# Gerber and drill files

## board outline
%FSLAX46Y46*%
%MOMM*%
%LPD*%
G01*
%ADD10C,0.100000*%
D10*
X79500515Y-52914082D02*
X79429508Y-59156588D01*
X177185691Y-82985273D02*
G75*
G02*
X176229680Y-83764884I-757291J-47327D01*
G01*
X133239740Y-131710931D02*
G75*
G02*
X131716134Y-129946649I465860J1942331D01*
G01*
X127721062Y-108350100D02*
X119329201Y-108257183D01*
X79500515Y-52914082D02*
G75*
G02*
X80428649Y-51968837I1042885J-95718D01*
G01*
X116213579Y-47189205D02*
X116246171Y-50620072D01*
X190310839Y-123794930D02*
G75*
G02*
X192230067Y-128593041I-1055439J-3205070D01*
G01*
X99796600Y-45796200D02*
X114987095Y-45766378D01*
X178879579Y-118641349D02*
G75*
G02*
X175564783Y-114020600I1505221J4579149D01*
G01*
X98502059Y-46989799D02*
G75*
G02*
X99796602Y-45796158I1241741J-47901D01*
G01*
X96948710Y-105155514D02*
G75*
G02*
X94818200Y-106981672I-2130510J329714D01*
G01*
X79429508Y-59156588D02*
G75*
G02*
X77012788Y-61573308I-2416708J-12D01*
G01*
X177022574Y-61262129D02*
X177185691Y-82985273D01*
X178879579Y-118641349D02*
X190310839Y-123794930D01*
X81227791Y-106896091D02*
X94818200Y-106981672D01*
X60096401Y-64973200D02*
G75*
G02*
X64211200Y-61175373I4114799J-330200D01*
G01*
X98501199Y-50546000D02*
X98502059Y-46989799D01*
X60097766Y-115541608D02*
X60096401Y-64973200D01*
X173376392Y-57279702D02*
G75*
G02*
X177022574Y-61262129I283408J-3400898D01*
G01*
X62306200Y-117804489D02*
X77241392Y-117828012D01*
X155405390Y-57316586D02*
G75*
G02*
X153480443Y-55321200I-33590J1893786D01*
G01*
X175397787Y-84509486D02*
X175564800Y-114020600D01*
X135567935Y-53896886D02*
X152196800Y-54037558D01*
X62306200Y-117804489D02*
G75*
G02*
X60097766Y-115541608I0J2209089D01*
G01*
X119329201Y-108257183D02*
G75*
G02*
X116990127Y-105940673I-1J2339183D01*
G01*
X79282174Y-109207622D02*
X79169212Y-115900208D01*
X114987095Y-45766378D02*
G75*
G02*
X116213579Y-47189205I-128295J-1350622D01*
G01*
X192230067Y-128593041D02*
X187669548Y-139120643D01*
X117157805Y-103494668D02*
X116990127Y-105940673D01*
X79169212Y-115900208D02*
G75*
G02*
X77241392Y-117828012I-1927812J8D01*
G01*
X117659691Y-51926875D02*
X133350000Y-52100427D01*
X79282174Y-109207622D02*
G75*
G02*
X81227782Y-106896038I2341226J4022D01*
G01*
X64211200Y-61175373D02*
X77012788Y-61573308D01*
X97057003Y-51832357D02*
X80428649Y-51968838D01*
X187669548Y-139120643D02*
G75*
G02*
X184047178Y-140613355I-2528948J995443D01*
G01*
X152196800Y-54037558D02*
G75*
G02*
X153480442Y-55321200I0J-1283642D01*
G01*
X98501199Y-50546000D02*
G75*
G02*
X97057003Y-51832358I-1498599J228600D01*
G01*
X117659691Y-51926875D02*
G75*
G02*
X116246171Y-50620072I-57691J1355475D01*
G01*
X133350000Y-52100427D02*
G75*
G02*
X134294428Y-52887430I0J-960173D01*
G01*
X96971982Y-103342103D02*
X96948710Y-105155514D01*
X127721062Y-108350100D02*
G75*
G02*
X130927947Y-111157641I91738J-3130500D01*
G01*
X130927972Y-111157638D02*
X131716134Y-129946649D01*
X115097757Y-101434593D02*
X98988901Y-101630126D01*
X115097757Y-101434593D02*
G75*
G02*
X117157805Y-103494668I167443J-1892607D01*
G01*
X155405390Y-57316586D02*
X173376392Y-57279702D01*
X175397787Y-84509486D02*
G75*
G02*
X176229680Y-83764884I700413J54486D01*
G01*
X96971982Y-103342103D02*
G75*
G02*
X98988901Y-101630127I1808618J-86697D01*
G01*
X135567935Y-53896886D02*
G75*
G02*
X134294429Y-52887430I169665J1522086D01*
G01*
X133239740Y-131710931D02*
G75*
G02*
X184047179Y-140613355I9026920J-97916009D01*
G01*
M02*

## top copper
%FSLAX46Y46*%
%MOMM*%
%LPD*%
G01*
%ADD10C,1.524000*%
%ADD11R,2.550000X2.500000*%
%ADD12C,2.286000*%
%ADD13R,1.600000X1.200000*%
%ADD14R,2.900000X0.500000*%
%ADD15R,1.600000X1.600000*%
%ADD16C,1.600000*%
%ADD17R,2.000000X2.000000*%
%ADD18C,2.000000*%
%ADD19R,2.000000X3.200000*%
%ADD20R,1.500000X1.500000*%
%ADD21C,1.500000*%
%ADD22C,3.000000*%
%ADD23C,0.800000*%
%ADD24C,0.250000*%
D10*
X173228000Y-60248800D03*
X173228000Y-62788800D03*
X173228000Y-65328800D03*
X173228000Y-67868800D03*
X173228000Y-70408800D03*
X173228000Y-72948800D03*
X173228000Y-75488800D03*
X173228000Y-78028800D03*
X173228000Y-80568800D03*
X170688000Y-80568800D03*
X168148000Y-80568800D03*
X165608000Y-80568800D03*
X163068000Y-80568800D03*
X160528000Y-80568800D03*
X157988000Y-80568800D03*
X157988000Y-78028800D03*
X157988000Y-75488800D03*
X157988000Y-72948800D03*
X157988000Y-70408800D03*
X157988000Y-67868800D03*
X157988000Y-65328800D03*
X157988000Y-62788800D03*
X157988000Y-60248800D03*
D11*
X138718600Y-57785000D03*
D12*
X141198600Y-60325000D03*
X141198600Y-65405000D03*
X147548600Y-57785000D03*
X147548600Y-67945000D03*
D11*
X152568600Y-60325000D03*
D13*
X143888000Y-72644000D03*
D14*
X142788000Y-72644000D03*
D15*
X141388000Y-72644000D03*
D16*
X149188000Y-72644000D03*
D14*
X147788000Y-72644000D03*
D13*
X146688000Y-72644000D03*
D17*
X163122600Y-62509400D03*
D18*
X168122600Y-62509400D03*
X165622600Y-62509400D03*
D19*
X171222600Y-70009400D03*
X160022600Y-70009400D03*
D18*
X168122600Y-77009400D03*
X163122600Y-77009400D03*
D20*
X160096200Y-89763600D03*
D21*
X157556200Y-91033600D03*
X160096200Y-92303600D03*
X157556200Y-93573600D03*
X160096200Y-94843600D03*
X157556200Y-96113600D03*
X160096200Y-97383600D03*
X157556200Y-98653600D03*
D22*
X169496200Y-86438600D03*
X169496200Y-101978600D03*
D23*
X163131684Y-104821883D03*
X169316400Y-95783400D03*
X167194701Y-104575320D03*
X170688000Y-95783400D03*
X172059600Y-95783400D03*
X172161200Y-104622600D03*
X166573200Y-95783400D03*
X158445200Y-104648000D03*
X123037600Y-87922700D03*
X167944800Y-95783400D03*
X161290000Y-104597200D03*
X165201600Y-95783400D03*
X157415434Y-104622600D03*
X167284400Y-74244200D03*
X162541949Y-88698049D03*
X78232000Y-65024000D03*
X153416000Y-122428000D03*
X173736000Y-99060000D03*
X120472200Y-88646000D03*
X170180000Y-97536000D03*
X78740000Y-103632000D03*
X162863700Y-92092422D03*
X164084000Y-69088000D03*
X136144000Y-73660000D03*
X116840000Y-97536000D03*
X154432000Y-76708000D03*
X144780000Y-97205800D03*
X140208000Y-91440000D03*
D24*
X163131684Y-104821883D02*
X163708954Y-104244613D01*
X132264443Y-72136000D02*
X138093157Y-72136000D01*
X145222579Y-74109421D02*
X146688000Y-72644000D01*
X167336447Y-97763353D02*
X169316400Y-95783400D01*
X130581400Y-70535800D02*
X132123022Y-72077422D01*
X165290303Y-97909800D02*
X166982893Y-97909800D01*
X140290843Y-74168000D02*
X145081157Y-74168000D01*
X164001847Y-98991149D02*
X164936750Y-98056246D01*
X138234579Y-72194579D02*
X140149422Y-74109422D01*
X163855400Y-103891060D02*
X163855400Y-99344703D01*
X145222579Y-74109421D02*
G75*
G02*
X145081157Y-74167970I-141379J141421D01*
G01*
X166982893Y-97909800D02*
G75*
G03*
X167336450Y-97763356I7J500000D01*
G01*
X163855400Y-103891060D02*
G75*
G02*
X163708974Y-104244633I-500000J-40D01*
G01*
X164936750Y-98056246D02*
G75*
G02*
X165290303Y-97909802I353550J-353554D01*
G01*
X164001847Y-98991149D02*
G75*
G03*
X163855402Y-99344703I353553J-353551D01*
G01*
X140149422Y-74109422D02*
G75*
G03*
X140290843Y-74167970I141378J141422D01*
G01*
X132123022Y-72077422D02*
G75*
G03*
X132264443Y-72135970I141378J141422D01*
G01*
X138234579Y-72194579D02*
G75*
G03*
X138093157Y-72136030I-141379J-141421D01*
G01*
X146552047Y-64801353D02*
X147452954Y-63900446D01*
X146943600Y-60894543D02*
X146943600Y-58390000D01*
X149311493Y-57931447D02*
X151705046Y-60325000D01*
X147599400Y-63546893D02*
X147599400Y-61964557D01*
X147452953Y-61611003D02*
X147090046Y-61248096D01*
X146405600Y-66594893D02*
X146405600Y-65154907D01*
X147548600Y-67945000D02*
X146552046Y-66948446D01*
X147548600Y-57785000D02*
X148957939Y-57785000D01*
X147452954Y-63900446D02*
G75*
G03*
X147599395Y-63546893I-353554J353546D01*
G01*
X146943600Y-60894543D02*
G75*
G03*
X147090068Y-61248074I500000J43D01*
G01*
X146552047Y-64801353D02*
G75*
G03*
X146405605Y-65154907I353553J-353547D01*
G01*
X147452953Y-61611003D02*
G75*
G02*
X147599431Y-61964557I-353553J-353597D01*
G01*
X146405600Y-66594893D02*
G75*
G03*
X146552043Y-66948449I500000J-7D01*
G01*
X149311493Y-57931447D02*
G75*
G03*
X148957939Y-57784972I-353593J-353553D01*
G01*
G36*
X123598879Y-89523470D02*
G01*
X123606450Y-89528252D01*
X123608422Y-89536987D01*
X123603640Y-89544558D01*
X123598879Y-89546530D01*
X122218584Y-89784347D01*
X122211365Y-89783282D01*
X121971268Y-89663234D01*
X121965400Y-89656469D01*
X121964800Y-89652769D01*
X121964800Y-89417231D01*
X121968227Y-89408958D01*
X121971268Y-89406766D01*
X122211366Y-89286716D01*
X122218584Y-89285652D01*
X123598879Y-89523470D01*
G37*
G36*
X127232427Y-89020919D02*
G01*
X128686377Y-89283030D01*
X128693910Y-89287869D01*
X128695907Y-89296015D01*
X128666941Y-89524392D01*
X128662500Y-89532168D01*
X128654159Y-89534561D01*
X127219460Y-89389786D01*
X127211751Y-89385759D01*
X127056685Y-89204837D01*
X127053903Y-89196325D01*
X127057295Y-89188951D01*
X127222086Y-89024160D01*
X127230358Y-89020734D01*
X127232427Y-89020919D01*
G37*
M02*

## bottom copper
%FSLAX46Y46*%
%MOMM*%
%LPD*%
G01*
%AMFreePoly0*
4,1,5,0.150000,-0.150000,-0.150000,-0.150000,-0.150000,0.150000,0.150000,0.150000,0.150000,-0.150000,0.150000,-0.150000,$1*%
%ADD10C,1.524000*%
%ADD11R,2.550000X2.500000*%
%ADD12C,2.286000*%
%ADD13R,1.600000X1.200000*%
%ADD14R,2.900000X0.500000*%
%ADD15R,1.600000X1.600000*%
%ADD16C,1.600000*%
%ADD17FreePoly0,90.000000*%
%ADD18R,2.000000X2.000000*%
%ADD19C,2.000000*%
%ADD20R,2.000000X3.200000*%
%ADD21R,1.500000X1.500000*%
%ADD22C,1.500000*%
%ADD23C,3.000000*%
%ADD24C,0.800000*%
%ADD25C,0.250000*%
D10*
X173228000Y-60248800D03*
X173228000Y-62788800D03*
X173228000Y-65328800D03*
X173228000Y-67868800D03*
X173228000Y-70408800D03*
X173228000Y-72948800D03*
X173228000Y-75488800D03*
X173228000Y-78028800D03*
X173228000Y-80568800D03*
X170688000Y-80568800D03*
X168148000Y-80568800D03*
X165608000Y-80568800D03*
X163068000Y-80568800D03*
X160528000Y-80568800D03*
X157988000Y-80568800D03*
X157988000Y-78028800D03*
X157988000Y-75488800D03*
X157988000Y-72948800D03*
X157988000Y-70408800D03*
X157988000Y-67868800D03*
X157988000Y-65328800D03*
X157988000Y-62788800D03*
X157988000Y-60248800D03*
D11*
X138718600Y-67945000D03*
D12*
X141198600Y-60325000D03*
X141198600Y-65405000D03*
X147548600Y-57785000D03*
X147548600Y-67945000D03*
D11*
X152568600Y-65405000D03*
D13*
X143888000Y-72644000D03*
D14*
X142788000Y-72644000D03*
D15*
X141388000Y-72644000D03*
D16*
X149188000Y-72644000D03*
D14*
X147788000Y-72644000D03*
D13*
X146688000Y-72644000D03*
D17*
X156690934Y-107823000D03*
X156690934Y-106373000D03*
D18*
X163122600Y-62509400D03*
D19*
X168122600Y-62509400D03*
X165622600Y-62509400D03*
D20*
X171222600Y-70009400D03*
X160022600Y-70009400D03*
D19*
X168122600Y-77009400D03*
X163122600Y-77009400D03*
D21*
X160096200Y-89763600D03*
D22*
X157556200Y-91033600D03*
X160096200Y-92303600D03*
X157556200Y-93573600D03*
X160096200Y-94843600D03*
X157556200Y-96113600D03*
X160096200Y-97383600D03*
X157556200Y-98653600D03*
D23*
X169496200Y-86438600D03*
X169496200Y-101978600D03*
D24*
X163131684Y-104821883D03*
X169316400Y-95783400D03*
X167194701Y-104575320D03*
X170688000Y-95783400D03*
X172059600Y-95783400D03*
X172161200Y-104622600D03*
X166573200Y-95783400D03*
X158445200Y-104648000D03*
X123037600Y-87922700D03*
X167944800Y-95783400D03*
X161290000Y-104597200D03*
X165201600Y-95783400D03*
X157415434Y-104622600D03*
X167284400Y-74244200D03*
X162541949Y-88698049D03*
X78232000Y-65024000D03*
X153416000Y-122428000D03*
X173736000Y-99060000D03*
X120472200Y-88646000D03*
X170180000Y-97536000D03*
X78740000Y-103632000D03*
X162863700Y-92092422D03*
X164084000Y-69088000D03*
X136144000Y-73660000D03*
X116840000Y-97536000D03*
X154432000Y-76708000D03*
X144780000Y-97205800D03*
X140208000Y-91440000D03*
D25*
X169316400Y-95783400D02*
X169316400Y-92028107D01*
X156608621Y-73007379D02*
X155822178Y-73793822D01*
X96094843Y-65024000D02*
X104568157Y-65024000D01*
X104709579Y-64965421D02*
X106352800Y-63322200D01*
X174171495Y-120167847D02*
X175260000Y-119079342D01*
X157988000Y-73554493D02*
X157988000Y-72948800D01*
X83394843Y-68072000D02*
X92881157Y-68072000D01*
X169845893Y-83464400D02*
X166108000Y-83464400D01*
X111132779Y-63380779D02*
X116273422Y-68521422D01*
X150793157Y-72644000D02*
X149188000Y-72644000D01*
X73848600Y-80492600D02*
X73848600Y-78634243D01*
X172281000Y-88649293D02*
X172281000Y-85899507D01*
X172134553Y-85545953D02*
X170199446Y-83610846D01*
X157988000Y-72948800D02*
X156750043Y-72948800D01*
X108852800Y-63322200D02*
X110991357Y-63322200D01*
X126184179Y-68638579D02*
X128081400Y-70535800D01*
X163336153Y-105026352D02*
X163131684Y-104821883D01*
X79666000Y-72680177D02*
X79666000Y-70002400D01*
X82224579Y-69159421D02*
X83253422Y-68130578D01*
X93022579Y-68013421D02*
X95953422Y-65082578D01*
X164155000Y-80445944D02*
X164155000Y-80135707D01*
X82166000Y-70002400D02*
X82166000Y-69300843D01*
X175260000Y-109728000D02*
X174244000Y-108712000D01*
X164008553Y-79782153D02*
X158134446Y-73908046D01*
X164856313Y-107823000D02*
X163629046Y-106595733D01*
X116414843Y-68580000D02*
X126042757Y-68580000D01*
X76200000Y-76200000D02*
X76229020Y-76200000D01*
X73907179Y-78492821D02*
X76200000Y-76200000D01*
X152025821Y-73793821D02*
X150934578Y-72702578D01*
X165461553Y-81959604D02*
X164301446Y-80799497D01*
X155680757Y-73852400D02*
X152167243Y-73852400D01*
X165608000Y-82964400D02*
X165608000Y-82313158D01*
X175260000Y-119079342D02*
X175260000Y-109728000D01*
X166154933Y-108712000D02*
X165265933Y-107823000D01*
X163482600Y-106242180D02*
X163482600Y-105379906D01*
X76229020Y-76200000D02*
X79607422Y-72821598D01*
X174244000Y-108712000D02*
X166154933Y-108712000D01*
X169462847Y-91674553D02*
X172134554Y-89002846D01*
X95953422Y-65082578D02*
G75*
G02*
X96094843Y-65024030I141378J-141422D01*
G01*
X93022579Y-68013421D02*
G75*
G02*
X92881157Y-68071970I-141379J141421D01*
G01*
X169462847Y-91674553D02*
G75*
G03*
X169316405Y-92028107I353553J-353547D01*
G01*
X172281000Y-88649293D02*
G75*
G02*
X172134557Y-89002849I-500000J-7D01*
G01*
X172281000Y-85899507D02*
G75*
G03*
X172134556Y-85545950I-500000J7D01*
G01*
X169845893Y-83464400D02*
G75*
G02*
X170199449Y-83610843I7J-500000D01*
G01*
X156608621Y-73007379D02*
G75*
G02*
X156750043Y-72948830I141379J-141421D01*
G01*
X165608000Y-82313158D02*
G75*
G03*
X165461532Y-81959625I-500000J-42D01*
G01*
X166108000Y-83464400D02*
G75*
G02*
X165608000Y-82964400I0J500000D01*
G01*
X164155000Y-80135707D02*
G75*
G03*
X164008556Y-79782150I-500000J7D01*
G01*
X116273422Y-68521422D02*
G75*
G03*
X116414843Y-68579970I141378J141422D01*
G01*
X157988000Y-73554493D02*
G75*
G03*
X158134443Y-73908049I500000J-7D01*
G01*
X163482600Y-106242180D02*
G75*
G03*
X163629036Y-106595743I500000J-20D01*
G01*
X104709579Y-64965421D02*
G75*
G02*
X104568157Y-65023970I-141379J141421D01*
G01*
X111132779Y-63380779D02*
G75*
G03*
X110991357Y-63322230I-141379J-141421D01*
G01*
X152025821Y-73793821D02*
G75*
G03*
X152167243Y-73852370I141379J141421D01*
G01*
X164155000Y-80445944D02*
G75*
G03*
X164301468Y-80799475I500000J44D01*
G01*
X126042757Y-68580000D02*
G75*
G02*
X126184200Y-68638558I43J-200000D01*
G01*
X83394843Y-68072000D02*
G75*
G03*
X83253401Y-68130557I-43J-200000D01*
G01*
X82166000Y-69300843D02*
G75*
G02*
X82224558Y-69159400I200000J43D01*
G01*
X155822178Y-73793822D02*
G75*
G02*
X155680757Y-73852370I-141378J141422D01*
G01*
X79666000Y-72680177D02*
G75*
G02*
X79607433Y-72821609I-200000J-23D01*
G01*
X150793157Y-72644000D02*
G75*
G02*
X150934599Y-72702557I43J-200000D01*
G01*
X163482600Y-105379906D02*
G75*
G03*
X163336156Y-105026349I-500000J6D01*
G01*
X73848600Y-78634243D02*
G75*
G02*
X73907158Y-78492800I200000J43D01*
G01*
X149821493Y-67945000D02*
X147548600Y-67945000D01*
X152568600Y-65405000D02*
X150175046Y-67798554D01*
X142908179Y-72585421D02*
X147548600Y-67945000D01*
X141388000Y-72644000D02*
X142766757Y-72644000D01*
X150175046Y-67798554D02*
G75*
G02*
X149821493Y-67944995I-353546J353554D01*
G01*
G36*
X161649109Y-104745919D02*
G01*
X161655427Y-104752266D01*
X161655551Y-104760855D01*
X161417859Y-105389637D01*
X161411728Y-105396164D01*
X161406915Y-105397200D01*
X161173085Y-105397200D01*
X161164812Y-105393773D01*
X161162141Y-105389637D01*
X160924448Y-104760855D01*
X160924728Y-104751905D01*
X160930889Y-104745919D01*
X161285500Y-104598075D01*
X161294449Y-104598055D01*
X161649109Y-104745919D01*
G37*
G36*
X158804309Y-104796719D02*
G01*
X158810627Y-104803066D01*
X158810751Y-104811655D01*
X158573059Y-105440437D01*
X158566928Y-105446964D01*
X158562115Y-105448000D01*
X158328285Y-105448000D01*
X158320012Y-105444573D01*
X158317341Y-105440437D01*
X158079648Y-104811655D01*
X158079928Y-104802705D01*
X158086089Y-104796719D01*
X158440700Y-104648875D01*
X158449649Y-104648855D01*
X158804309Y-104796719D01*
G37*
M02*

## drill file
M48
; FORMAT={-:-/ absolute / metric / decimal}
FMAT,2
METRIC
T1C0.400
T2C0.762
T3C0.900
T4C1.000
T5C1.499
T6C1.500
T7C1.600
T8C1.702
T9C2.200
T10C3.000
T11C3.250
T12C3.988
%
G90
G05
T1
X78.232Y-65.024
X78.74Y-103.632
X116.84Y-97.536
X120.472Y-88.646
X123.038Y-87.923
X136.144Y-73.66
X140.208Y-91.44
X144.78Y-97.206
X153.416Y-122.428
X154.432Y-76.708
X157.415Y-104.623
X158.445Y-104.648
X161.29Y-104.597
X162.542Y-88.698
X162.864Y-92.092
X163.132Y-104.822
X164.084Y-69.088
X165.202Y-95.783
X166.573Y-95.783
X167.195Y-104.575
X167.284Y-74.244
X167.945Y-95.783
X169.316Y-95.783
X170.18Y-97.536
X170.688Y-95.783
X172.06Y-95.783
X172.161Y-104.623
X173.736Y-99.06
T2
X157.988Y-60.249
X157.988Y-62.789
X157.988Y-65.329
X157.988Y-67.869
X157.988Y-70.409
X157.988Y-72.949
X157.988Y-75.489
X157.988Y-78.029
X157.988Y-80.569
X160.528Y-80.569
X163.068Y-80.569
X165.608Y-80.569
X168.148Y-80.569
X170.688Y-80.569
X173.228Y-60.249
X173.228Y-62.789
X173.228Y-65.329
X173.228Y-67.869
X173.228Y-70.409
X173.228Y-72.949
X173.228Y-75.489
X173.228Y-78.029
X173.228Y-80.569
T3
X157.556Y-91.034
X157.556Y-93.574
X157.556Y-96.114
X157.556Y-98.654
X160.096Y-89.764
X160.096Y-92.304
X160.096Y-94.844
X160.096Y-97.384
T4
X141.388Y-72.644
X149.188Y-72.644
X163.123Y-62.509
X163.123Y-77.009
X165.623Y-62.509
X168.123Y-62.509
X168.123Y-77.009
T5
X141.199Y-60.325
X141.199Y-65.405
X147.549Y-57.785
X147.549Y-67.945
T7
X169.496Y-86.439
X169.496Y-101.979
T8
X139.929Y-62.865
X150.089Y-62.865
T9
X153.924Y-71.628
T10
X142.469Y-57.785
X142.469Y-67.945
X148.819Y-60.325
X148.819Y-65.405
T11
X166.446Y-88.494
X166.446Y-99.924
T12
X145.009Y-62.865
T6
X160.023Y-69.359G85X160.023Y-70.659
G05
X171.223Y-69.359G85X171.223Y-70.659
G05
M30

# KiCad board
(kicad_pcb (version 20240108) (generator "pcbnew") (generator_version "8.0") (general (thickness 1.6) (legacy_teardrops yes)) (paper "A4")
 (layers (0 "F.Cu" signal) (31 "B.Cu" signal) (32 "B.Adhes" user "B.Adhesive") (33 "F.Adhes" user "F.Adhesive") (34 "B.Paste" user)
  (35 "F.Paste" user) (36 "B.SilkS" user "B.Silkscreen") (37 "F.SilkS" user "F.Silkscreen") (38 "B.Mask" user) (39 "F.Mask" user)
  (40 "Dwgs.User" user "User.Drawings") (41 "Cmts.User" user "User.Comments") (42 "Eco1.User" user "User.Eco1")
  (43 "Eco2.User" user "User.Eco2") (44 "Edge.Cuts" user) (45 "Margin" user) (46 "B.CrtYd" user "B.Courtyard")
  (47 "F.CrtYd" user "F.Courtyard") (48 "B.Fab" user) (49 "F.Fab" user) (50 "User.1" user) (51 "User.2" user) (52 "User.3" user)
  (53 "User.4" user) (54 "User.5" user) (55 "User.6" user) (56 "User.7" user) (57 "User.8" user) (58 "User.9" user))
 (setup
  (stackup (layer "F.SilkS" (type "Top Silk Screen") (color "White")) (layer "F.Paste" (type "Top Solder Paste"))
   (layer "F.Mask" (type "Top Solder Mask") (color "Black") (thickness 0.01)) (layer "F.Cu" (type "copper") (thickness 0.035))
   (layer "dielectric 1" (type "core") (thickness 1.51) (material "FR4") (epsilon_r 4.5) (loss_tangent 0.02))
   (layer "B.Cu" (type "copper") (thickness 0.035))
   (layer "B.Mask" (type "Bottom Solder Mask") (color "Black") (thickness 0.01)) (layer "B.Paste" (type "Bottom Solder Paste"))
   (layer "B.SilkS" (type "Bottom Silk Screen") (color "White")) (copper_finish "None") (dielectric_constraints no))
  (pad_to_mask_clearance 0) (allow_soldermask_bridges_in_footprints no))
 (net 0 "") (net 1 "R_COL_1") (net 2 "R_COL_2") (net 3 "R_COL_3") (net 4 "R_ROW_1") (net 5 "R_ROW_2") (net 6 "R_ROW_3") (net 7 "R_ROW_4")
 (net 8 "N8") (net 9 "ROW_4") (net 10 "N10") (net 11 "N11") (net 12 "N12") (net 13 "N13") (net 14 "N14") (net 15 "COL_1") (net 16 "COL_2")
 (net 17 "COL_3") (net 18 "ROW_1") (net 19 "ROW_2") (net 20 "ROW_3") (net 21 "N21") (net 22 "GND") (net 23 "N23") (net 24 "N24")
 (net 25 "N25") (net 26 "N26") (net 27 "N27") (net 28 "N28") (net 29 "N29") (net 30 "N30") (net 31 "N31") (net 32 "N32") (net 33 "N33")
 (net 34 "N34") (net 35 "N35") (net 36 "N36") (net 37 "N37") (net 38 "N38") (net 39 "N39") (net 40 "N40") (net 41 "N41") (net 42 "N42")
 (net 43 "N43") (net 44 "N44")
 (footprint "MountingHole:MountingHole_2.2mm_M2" (layer "F.Cu") (at 153.924 71.628)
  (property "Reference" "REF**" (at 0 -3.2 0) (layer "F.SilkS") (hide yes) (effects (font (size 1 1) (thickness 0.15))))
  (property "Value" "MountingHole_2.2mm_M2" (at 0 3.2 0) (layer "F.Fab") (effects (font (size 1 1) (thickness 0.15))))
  (pad "" np_thru_hole circle (at 0 0) (size 2.2 2.2) (drill 2.2) (layers "*.Cu" "*.Mask")))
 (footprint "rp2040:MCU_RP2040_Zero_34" (layer "F.Cu") (at 163.068 67.8688)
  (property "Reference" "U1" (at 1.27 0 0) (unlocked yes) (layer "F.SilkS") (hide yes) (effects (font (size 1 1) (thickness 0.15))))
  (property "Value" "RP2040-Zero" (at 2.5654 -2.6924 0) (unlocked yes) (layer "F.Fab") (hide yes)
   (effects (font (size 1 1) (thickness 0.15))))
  (pad "0" thru_hole circle (at 10.16 -7.62) (size 1.524 1.524) (drill 0.762) (layers "*.Cu" "*.Mask") (remove_unused_layers no)
   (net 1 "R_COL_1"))
  (pad "1" thru_hole circle (at 10.16 -5.08) (size 1.524 1.524) (drill 0.762) (layers "*.Cu" "*.Mask") (remove_unused_layers no)
   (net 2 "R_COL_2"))
  (pad "2" thru_hole circle (at 10.16 -2.54) (size 1.524 1.524) (drill 0.762) (layers "*.Cu" "*.Mask") (remove_unused_layers no)
   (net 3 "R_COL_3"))
  (pad "3" thru_hole circle (at 10.16 0) (size 1.524 1.524) (drill 0.762) (layers "*.Cu" "*.Mask") (remove_unused_layers no)
   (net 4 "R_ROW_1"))
  (pad "4" thru_hole circle (at 10.16 2.54) (size 1.524 1.524) (drill 0.762) (layers "*.Cu" "*.Mask") (remove_unused_layers no)
   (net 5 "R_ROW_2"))
  (pad "5" thru_hole circle (at 10.16 5.08) (size 1.524 1.524) (drill 0.762) (layers "*.Cu" "*.Mask") (remove_unused_layers no)
   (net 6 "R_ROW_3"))
  (pad "6" thru_hole circle (at 10.16 7.62) (size 1.524 1.524) (drill 0.762) (layers "*.Cu" "*.Mask") (remove_unused_layers no)
   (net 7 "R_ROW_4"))
  (pad "7" thru_hole circle (at 10.16 10.16) (size 1.524 1.524) (drill 0.762) (layers "*.Cu" "*.Mask") (remove_unused_layers no)
   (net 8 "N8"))
  (pad "8" thru_hole circle (at 10.16 12.7) (size 1.524 1.524) (drill 0.762) (layers "*.Cu" "*.Mask") (remove_unused_layers no)
   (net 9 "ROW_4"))
  (pad "9" thru_hole circle (at 7.62 12.7) (size 1.524 1.524) (drill 0.762) (layers "*.Cu" "*.Mask") (remove_unused_layers no)
   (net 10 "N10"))
  (pad "10" thru_hole circle (at 5.08 12.7) (size 1.524 1.524) (drill 0.762) (layers "*.Cu" "*.Mask") (remove_unused_layers no)
   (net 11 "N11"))
  (pad "11" thru_hole circle (at 2.54 12.7) (size 1.524 1.524) (drill 0.762) (layers "*.Cu" "*.Mask") (remove_unused_layers no)
   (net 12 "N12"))
  (pad "12" thru_hole circle (at 0 12.7) (size 1.524 1.524) (drill 0.762) (layers "*.Cu" "*.Mask") (remove_unused_layers no) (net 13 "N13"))
  (pad "13" thru_hole circle (at -2.54 12.7) (size 1.524 1.524) (drill 0.762) (layers "*.Cu" "*.Mask") (remove_unused_layers no)
   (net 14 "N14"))
  (pad "14" thru_hole circle (at -5.08 12.7) (size 1.524 1.524) (drill 0.762) (layers "*.Cu" "*.Mask") (remove_unused_layers no)
   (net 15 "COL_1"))
  (pad "15" thru_hole circle (at -5.08 10.16) (size 1.524 1.524) (drill 0.762) (layers "*.Cu" "*.Mask") (remove_unused_layers no)
   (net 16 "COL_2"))
  (pad "26" thru_hole circle (at -5.08 7.62) (size 1.524 1.524) (drill 0.762) (layers "*.Cu" "*.Mask") (remove_unused_layers no)
   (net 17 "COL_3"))
  (pad "27" thru_hole circle (at -5.08 5.08) (size 1.524 1.524) (drill 0.762) (layers "*.Cu" "*.Mask") (remove_unused_layers no)
   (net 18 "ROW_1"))
  (pad "28" thru_hole circle (at -5.08 2.54) (size 1.524 1.524) (drill 0.762) (layers "*.Cu" "*.Mask") (remove_unused_layers no)
   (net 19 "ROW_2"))
  (pad "29" thru_hole circle (at -5.08 0) (size 1.524 1.524) (drill 0.762) (layers "*.Cu" "*.Mask") (remove_unused_layers no)
   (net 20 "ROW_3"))
  (pad "30" thru_hole circle (at -5.08 -2.54) (size 1.524 1.524) (drill 0.762) (layers "*.Cu" "*.Mask") (remove_unused_layers no)
   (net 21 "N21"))
  (pad "31" thru_hole circle (at -5.08 -5.08) (size 1.524 1.524) (drill 0.762) (layers "*.Cu" "*.Mask") (remove_unused_layers no)
   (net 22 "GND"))
  (pad "32" thru_hole circle (at -5.08 -7.62) (size 1.524 1.524) (drill 0.762) (layers "*.Cu" "*.Mask") (remove_unused_layers no)
   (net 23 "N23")))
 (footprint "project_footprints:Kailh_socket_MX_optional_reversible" (layer "F.Cu") (at 145.0086 62.865)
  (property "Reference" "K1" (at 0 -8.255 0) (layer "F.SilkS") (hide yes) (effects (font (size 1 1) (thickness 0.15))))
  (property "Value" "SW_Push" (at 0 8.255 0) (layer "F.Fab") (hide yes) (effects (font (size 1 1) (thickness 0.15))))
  (pad "" np_thru_hole circle (at -5.08 0) (size 1.7018 1.7018) (drill 1.7018) (layers "*.Cu" "*.Mask"))
  (pad "" np_thru_hole circle (at -2.54 -5.08) (size 3 3) (drill 3) (layers "*.Cu" "*.Mask"))
  (pad "" np_thru_hole circle (at -2.54 5.08) (size 3 3) (drill 3) (layers "*.Cu" "*.Mask"))
  (pad "" np_thru_hole circle (at 0 0) (size 3.9878 3.9878) (drill 3.9878) (layers "*.Cu" "*.Mask"))
  (pad "" np_thru_hole circle (at 3.81 -2.54) (size 3 3) (drill 3) (layers "*.Cu" "*.Mask"))
  (pad "" np_thru_hole circle (at 3.81 2.54) (size 3 3) (drill 3) (layers "*.Cu" "*.Mask"))
  (pad "" np_thru_hole circle (at 5.08 0) (size 1.7018 1.7018) (drill 1.7018) (layers "*.Cu" "*.Mask"))
  (pad "1" smd rect (at -6.29 -5.08) (size 2.55 2.5) (layers "F.Cu" "F.Paste" "F.Mask") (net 15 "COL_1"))
  (pad "1" smd rect (at -6.29 5.08) (size 2.55 2.5) (layers "B.Cu" "B.Paste" "B.Mask") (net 15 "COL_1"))
  (pad "1" thru_hole circle (at -3.81 -2.54) (size 2.286 2.286) (drill 1.4986) (layers "*.Cu" "*.Mask") (remove_unused_layers no)
   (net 15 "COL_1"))
  (pad "1" thru_hole circle (at -3.81 2.54) (size 2.286 2.286) (drill 1.4986) (layers "*.Cu" "*.Mask") (remove_unused_layers no)
   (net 15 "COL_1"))
  (pad "2" thru_hole circle (at 2.54 -5.08) (size 2.286 2.286) (drill 1.4986) (layers "*.Cu" "*.Mask") (remove_unused_layers no)
   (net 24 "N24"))
  (pad "2" thru_hole circle (at 2.54 5.08) (size 2.286 2.286) (drill 1.4986) (layers "*.Cu" "*.Mask") (remove_unused_layers no)
   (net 24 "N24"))
  (pad "2" smd rect (at 7.56 -2.54) (size 2.55 2.5) (layers "F.Cu" "F.Paste" "F.Mask") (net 24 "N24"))
  (pad "2" smd rect (at 7.56 2.54) (size 2.55 2.5) (layers "B.Cu" "B.Paste" "B.Mask") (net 24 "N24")))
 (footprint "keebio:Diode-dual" (layer "F.Cu") (at 145.288 72.644 180)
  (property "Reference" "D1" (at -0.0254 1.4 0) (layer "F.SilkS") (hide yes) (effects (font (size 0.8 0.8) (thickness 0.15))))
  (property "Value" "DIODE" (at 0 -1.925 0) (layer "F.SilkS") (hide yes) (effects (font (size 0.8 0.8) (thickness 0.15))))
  (pad "1" smd rect (at 1.4 0 180) (size 1.6 1.2) (layers "F.Cu" "F.Paste" "F.Mask") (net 24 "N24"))
  (pad "1" smd rect (at 1.4 0 180) (size 1.6 1.2) (layers "B.Cu" "B.Paste" "B.Mask") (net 24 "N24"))
  (pad "1" smd rect (at 2.5 0 180) (size 2.9 0.5) (layers "F.Cu") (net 24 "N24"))
  (pad "1" smd rect (at 2.5 0 180) (size 2.9 0.5) (layers "B.Cu") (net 24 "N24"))
  (pad "1" thru_hole rect (at 3.9 0 180) (size 1.6 1.6) (drill 1) (layers "*.Cu" "*.Mask" "F.SilkS") (remove_unused_layers no)
   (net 24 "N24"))
  (pad "2" thru_hole circle (at -3.9 0 180) (size 1.6 1.6) (drill 1) (layers "*.Cu" "*.Mask" "F.SilkS") (remove_unused_layers no)
   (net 18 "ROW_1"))
  (pad "2" smd rect (at -2.5 0 180) (size 2.9 0.5) (layers "F.Cu") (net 18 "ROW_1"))
  (pad "2" smd rect (at -2.5 0 180) (size 2.9 0.5) (layers "B.Cu") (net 18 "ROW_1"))
  (pad "2" smd rect (at -1.4 0 180) (size 1.6 1.2) (layers "F.Cu" "F.Paste" "F.Mask") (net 18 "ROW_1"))
  (pad "2" smd rect (at -1.4 0 180) (size 1.6 1.2) (layers "B.Cu" "B.Paste" "B.Mask") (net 18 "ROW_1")))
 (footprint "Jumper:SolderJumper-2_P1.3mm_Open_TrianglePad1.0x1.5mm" (layer "B.Cu") (at 156.690934 107.098 90)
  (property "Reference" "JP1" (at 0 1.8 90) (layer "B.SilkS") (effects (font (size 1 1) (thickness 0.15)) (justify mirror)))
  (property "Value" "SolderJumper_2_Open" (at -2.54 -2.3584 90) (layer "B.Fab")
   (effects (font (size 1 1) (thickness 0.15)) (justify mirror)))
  (pad "1" smd custom (at -0.725 0 90) (size 0.3 0.3) (layers "B.Cu" "B.Mask") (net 15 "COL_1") (zone_connect 2) (thermal_bridge_angle 45)
   (options (clearance outline) (anchor rect)) (primitives))
  (pad "2" smd custom (at 0.725 0 90) (size 0.3 0.3) (layers "B.Cu" "B.Mask") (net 1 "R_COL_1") (zone_connect 2) (thermal_bridge_angle 45)
   (options (clearance outline) (anchor rect)) (primitives)))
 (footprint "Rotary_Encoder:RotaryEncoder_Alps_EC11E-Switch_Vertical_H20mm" (layer "B.Cu") (at 163.1226 62.5094 -90)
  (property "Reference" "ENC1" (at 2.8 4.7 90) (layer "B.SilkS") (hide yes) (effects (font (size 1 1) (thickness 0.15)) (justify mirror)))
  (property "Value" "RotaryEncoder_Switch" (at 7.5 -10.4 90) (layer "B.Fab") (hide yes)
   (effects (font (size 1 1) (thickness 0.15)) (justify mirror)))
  (pad "A" thru_hole rect (at 0 0 270) (size 2 2) (drill 1) (layers "*.Cu" "*.Mask") (remove_unused_layers no) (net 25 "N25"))
  (pad "B" thru_hole circle (at 0 -5 270) (size 2 2) (drill 1) (layers "*.Cu" "*.Mask") (remove_unused_layers no) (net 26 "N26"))
  (pad "C" thru_hole circle (at 0 -2.5 270) (size 2 2) (drill 1) (layers "*.Cu" "*.Mask") (remove_unused_layers no) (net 9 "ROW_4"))
  (pad "MP" thru_hole rect (at 7.5 -8.1 270) (size 3.2 2) (drill oval 2.8 1.5) (layers "*.Cu" "*.Mask") (remove_unused_layers no))
  (pad "MP" thru_hole rect (at 7.5 3.1 270) (size 3.2 2) (drill oval 2.8 1.5) (layers "*.Cu" "*.Mask") (remove_unused_layers no))
  (pad "S1" thru_hole circle (at 14.5 -5 270) (size 2 2) (drill 1) (layers "*.Cu" "*.Mask") (remove_unused_layers no) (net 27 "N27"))
  (pad "S2" thru_hole circle (at 14.5 0 270) (size 2 2) (drill 1) (layers "*.Cu" "*.Mask") (remove_unused_layers no) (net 9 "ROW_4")))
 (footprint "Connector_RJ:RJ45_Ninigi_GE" (layer "B.Cu") (at 160.0962 89.7636 -90)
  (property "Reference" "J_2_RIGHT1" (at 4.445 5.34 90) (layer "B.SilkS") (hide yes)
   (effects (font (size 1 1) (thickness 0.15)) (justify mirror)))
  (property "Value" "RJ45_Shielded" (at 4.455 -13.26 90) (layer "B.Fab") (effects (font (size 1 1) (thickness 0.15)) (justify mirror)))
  (pad "" np_thru_hole circle (at -1.27 -6.35 270) (size 3.25 3.25) (drill 3.25) (layers "*.Cu" "*.Mask"))
  (pad "" np_thru_hole circle (at 10.16 -6.35 90) (size 3.25 3.25) (drill 3.25) (layers "*.Cu" "*.Mask"))
  (pad "1" thru_hole rect (at 0 0 90) (size 1.5 1.5) (drill 0.9) (layers "*.Cu" "*.Mask") (remove_unused_layers no) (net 22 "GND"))
  (pad "2" thru_hole circle (at 1.27 2.54 90) (size 1.5 1.5) (drill 0.9) (layers "*.Cu" "*.Mask") (remove_unused_layers no)
   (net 7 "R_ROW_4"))
  (pad "3" thru_hole circle (at 2.54 0 90) (size 1.5 1.5) (drill 0.9) (layers "*.Cu" "*.Mask") (remove_unused_layers no) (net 6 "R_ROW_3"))
  (pad "4" thru_hole circle (at 3.81 2.54 90) (size 1.5 1.5) (drill 0.9) (layers "*.Cu" "*.Mask") (remove_unused_layers no)
   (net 5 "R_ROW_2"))
  (pad "5" thru_hole circle (at 5.08 0 90) (size 1.5 1.5) (drill 0.9) (layers "*.Cu" "*.Mask") (remove_unused_layers no) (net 4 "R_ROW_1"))
  (pad "6" thru_hole circle (at 6.35 2.54 90) (size 1.5 1.5) (drill 0.9) (layers "*.Cu" "*.Mask") (remove_unused_layers no)
   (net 3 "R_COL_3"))
  (pad "7" thru_hole circle (at 7.62 0 90) (size 1.5 1.5) (drill 0.9) (layers "*.Cu" "*.Mask") (remove_unused_layers no) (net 2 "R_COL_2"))
  (pad "8" thru_hole circle (at 8.89 2.54 90) (size 1.5 1.5) (drill 0.9) (layers "*.Cu" "*.Mask") (remove_unused_layers no)
   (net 1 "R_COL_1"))
  (pad "SH" thru_hole circle (at -3.325 -9.4 270) (size 3 3) (drill 1.6) (layers "*.Cu" "*.Mask") (remove_unused_layers no) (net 22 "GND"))
  (pad "SH" thru_hole circle (at 12.215 -9.4 90) (size 3 3) (drill 1.6) (layers "*.Cu" "*.Mask") (remove_unused_layers no) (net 22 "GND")))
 (gr_line (start 79.500515 52.914082) (end 79.429508 59.156588) (stroke (width 0.1) (type solid)) (layer "Edge.Cuts"))
 (gr_arc (start 177.185691 82.985273) (mid 176.90793 83.620631) (end 176.22968 83.764884) (stroke (width 0.1) (type solid))
  (layer "Edge.Cuts"))
 (gr_arc (start 133.23974 131.710931) (mid 132.19387 131.074106) (end 131.716134 129.946649) (stroke (width 0.1) (type solid))
  (layer "Edge.Cuts"))
 (gr_line (start 127.721062 108.3501) (end 119.329201 108.257183) (stroke (width 0.1) (type solid)) (layer "Edge.Cuts"))
 (gr_arc (start 79.500515 52.914082) (mid 79.796137 52.276064) (end 80.428649 51.968838) (stroke (width 0.1) (type solid))
  (layer "Edge.Cuts"))
 (gr_line (start 116.213579 47.189205) (end 116.246171 50.620072) (stroke (width 0.1) (type solid)) (layer "Edge.Cuts"))
 (gr_arc (start 190.310839 123.79493) (mid 192.388435 125.746797) (end 192.230067 128.593041) (stroke (width 0.1) (type solid))
  (layer "Edge.Cuts"))
 (gr_line (start 99.7966 45.7962) (end 114.987095 45.766378) (stroke (width 0.1) (type solid)) (layer "Edge.Cuts"))
 (gr_arc (start 178.879579 118.641349) (mid 176.468183 116.871883) (end 175.5648 114.0206) (stroke (width 0.1) (type solid))
  (layer "Edge.Cuts"))
 (gr_arc (start 98.502059 46.989799) (mid 98.901429 46.124135) (end 99.7966 45.7962) (stroke (width 0.1) (type solid)) (layer "Edge.Cuts"))
 (gr_arc (start 96.94871 105.155514) (mid 96.221226 106.462658) (end 94.8182 106.981672) (stroke (width 0.1) (type solid))
  (layer "Edge.Cuts"))
 (gr_arc (start 79.429508 59.156588) (mid 78.721671 60.865471) (end 77.012788 61.573308) (stroke (width 0.1) (type solid))
  (layer "Edge.Cuts"))
 (gr_line (start 177.022574 61.262129) (end 177.185691 82.985273) (stroke (width 0.1) (type solid)) (layer "Edge.Cuts"))
 (gr_line (start 178.879579 118.641349) (end 190.310839 123.79493) (stroke (width 0.1) (type solid)) (layer "Edge.Cuts"))
 (gr_line (start 81.227791 106.896091) (end 94.8182 106.981672) (stroke (width 0.1) (type default)) (layer "Edge.Cuts"))
 (gr_arc (start 60.096401 64.9732) (mid 61.411421 62.269947) (end 64.2112 61.175373) (stroke (width 0.1) (type solid)) (layer "Edge.Cuts"))
 (gr_line (start 98.501199 50.546) (end 98.502059 46.989799) (stroke (width 0.1) (type default)) (layer "Edge.Cuts"))
 (gr_line (start 60.097766 115.541608) (end 60.096401 64.9732) (stroke (width 0.1) (type solid)) (layer "Edge.Cuts"))
 (gr_arc (start 173.376392 57.279702) (mid 176.176853 58.376067) (end 177.022574 61.262129) (stroke (width 0.1) (type solid))
  (layer "Edge.Cuts"))
 (gr_line (start 62.3062 117.804489) (end 77.241392 117.828012) (stroke (width 0.1) (type default)) (layer "Edge.Cuts"))
 (gr_arc (start 155.40539 57.316586) (mid 154.008636 56.737843) (end 153.480443 55.3212) (stroke (width 0.1) (type solid))
  (layer "Edge.Cuts"))
 (gr_line (start 175.397787 84.509486) (end 175.5648 114.0206) (stroke (width 0.1) (type solid)) (layer "Edge.Cuts"))
 (gr_line (start 135.567935 53.896886) (end 152.1968 54.037558) (stroke (width 0.1) (type solid)) (layer "Edge.Cuts"))
 (gr_arc (start 62.3062 117.804489) (mid 60.725234 117.138326) (end 60.097766 115.541608) (stroke (width 0.1) (type solid))
  (layer "Edge.Cuts"))
 (gr_arc (start 119.329201 108.257183) (mid 117.683184 107.580049) (end 116.990127 105.940673) (stroke (width 0.1) (type solid))
  (layer "Edge.Cuts"))
 (gr_line (start 79.282174 109.207622) (end 79.169212 115.900208) (stroke (width 0.1) (type solid)) (layer "Edge.Cuts"))
 (gr_arc (start 114.987095 45.766378) (mid 115.886412 46.231193) (end 116.213579 47.189205) (stroke (width 0.1) (type solid))
  (layer "Edge.Cuts"))
 (gr_line (start 192.230067 128.593041) (end 187.669548 139.120643) (stroke (width 0.1) (type solid)) (layer "Edge.Cuts"))
 (gr_line (start 117.157805 103.494668) (end 116.990127 105.940673) (stroke (width 0.1) (type default)) (layer "Edge.Cuts"))
 (gr_arc (start 79.169212 115.900208) (mid 78.604563 117.263375) (end 77.241392 117.828012) (stroke (width 0.1) (type solid))
  (layer "Edge.Cuts"))
 (gr_line (start 117.659691 51.926875) (end 133.35 52.100427) (stroke (width 0.1) (type solid)) (layer "Edge.Cuts"))
 (gr_arc (start 79.282174 109.207622) (mid 79.8322 107.696) (end 81.227791 106.896091) (stroke (width 0.1) (type solid)) (layer "Edge.Cuts"))
 (gr_line (start 64.2112 61.175373) (end 77.012788 61.573308) (stroke (width 0.1) (type solid)) (layer "Edge.Cuts"))
 (gr_line (start 97.057003 51.832357) (end 80.428649 51.968838) (stroke (width 0.1) (type default)) (layer "Edge.Cuts"))
 (gr_arc (start 187.669548 139.120643) (mid 186.176086 140.638018) (end 184.047178 140.613355) (stroke (width 0.1) (type solid))
  (layer "Edge.Cuts"))
 (gr_arc (start 152.1968 54.037558) (mid 153.104472 54.413528) (end 153.480442 55.3212) (stroke (width 0.1) (type solid))
  (layer "Edge.Cuts"))
 (gr_arc (start 98.501199 50.546) (mid 98.010882 51.4494) (end 97.057003 51.832357) (stroke (width 0.1) (type solid)) (layer "Edge.Cuts"))
 (gr_arc (start 117.659691 51.926875) (mid 116.681009 51.567601) (end 116.246171 50.620072) (stroke (width 0.1) (type solid))
  (layer "Edge.Cuts"))
 (gr_arc (start 133.35 52.100427) (mid 133.964678 52.322967) (end 134.294428 52.88743) (stroke (width 0.1) (type solid)) (layer "Edge.Cuts"))
 (gr_line (start 96.971982 103.342103) (end 96.94871 105.155514) (stroke (width 0.1) (type default)) (layer "Edge.Cuts"))
 (gr_arc (start 127.721062 108.3501) (mid 129.875764 109.124199) (end 130.927972 111.157638) (stroke (width 0.1) (type solid))
  (layer "Edge.Cuts"))
 (gr_line (start 130.927972 111.157638) (end 131.716134 129.946649) (stroke (width 0.1) (type solid)) (layer "Edge.Cuts"))
 (gr_line (start 115.097757 101.434593) (end 98.988901 101.630126) (stroke (width 0.1) (type solid)) (layer "Edge.Cuts"))
 (gr_arc (start 115.097757 101.434593) (mid 116.608711 101.983706) (end 117.157805 103.494668) (stroke (width 0.1) (type solid))
  (layer "Edge.Cuts"))
 (gr_line (start 155.40539 57.316586) (end 173.376392 57.279702) (stroke (width 0.1) (type solid)) (layer "Edge.Cuts"))
 (gr_arc (start 175.397787 84.509486) (mid 175.629661 83.931533) (end 176.22968 83.764884) (stroke (width 0.1) (type solid))
  (layer "Edge.Cuts"))
 (gr_arc (start 96.971982 103.342103) (mid 97.608862 102.048349) (end 98.988901 101.630126) (stroke (width 0.1) (type solid))
  (layer "Edge.Cuts"))
 (gr_arc (start 135.567935 53.896886) (mid 134.786253 53.574997) (end 134.294429 52.88743) (stroke (width 0.1) (type solid))
  (layer "Edge.Cuts"))
 (gr_arc (start 133.23974 131.710931) (mid 159.237601 132.771289) (end 184.047178 140.613356) (stroke (width 0.1) (type solid))
  (layer "Edge.Cuts"))
 (segment (start 163.131684 104.821883) (end 163.708954 104.244613) (width 0.25) (layer "F.Cu") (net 18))
 (segment (start 132.264443 72.136) (end 138.093157 72.136) (width 0.25) (layer "F.Cu") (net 18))
 (segment (start 145.222579 74.109421) (end 146.688 72.644) (width 0.25) (layer "F.Cu") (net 18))
 (segment (start 167.336447 97.763353) (end 169.3164 95.7834) (width 0.25) (layer "F.Cu") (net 18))
 (segment (start 130.5814 70.5358) (end 132.123022 72.077422) (width 0.25) (layer "F.Cu") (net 18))
 (segment (start 165.290303 97.9098) (end 166.982893 97.9098) (width 0.25) (layer "F.Cu") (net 18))
 (segment (start 140.290843 74.168) (end 145.081157 74.168) (width 0.25) (layer "F.Cu") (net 18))
 (segment (start 164.001847 98.991149) (end 164.93675 98.056246) (width 0.25) (layer "F.Cu") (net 18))
 (segment (start 138.234579 72.194579) (end 140.149422 74.109422) (width 0.25) (layer "F.Cu") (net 18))
 (segment (start 163.8554 103.89106) (end 163.8554 99.344703) (width 0.25) (layer "F.Cu") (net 18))
 (via (at 163.131684 104.821883) (size 0.8) (drill 0.4) (layers "F.Cu" "B.Cu") (free yes) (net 18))
 (via (at 169.3164 95.7834) (size 0.8) (drill 0.4) (layers "F.Cu" "B.Cu") (free yes) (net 18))
 (arc (start 145.222579 74.109421) (mid 145.157694 74.152776) (end 145.081157 74.168) (width 0.25) (layer "F.Cu") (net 18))
 (arc (start 166.982893 97.9098) (mid 167.174235 97.87174) (end 167.336447 97.763353) (width 0.25) (layer "F.Cu") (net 18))
 (arc (start 163.8554 103.89106) (mid 163.81734 104.082401) (end 163.708954 104.244613) (width 0.25) (layer "F.Cu") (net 18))
 (arc (start 164.93675 98.056246) (mid 165.098962 97.94786) (end 165.290303 97.9098) (width 0.25) (layer "F.Cu") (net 18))
 (arc (start 164.001847 98.991149) (mid 163.89346 99.153361) (end 163.8554 99.344703) (width 0.25) (layer "F.Cu") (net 18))
 (arc (start 140.149422 74.109422) (mid 140.214307 74.152776) (end 140.290843 74.168) (width 0.25) (layer "F.Cu") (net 18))
 (arc (start 132.123022 72.077422) (mid 132.187907 72.120776) (end 132.264443 72.136) (width 0.25) (layer "F.Cu") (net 18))
 (arc (start 138.234579 72.194579) (mid 138.169694 72.151224) (end 138.093157 72.136) (width 0.25) (layer "F.Cu") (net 18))
 (segment (start 169.3164 95.7834) (end 169.3164 92.028107) (width 0.25) (layer "B.Cu") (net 18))
 (segment (start 156.608621 73.007379) (end 155.822178 73.793822) (width 0.25) (layer "B.Cu") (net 18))
 (segment (start 96.094843 65.024) (end 104.568157 65.024) (width 0.25) (layer "B.Cu") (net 18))
 (segment (start 104.709579 64.965421) (end 106.3528 63.3222) (width 0.25) (layer "B.Cu") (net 18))
 (segment (start 174.171495 120.167847) (end 175.26 119.079342) (width 0.25) (layer "B.Cu") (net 18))
 (segment (start 157.988 73.554493) (end 157.988 72.9488) (width 0.25) (layer "B.Cu") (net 18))
 (segment (start 83.394843 68.072) (end 92.881157 68.072) (width 0.25) (layer "B.Cu") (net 18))
 (segment (start 169.845893 83.4644) (end 166.108 83.4644) (width 0.25) (layer "B.Cu") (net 18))
 (segment (start 111.132779 63.380779) (end 116.273422 68.521422) (width 0.25) (layer "B.Cu") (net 18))
 (segment (start 150.793157 72.644) (end 149.188 72.644) (width 0.25) (layer "B.Cu") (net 18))
 (segment (start 73.8486 80.4926) (end 73.8486 78.634243) (width 0.25) (layer "B.Cu") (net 18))
 (segment (start 172.281 88.649293) (end 172.281 85.899507) (width 0.25) (layer "B.Cu") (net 18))
 (segment (start 172.134553 85.545953) (end 170.199446 83.610846) (width 0.25) (layer "B.Cu") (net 18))
 (segment (start 157.988 72.9488) (end 156.750043 72.9488) (width 0.25) (layer "B.Cu") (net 18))
 (segment (start 108.8528 63.3222) (end 110.991357 63.3222) (width 0.25) (layer "B.Cu") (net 18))
 (segment (start 126.184179 68.638579) (end 128.0814 70.5358) (width 0.25) (layer "B.Cu") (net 18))
 (segment (start 163.336153 105.026352) (end 163.131684 104.821883) (width 0.25) (layer "B.Cu") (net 18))
 (segment (start 79.666 72.680177) (end 79.666 70.0024) (width 0.25) (layer "B.Cu") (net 18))
 (segment (start 82.224579 69.159421) (end 83.253422 68.130578) (width 0.25) (layer "B.Cu") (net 18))
 (segment (start 93.022579 68.013421) (end 95.953422 65.082578) (width 0.25) (layer "B.Cu") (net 18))
 (segment (start 164.155 80.445944) (end 164.155 80.135707) (width 0.25) (layer "B.Cu") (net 18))
 (segment (start 82.166 70.0024) (end 82.166 69.300843) (width 0.25) (layer "B.Cu") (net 18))
 (segment (start 175.26 109.728) (end 174.244 108.712) (width 0.25) (layer "B.Cu") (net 18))
 (segment (start 164.008553 79.782153) (end 158.134446 73.908046) (width 0.25) (layer "B.Cu") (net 18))
 (segment (start 164.856313 107.823) (end 163.629046 106.595733) (width 0.25) (layer "B.Cu") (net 18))
 (segment (start 116.414843 68.58) (end 126.042757 68.58) (width 0.25) (layer "B.Cu") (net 18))
 (segment (start 76.2 76.2) (end 76.22902 76.2) (width 0.25) (layer "B.Cu") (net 18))
 (segment (start 73.907179 78.492821) (end 76.2 76.2) (width 0.25) (layer "B.Cu") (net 18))
 (segment (start 152.025821 73.793821) (end 150.934578 72.702578) (width 0.25) (layer "B.Cu") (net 18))
 (segment (start 165.461553 81.959604) (end 164.301446 80.799497) (width 0.25) (layer "B.Cu") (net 18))
 (segment (start 155.680757 73.8524) (end 152.167243 73.8524) (width 0.25) (layer "B.Cu") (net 18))
 (segment (start 165.608 82.9644) (end 165.608 82.313158) (width 0.25) (layer "B.Cu") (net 18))
 (segment (start 175.26 119.079342) (end 175.26 109.728) (width 0.25) (layer "B.Cu") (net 18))
 (segment (start 166.154933 108.712) (end 165.265933 107.823) (width 0.25) (layer "B.Cu") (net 18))
 (segment (start 163.4826 106.24218) (end 163.4826 105.379906) (width 0.25) (layer "B.Cu") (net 18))
 (segment (start 76.22902 76.2) (end 79.607422 72.821598) (width 0.25) (layer "B.Cu") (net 18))
 (segment (start 174.244 108.712) (end 166.154933 108.712) (width 0.25) (layer "B.Cu") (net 18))
 (segment (start 169.462847 91.674553) (end 172.134554 89.002846) (width 0.25) (layer "B.Cu") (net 18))
 (arc (start 95.953422 65.082578) (mid 96.018307 65.039224) (end 96.094843 65.024) (width 0.25) (layer "B.Cu") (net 18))
 (arc (start 93.022579 68.013421) (mid 92.957694 68.056776) (end 92.881157 68.072) (width 0.25) (layer "B.Cu") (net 18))
 (arc (start 169.462847 91.674553) (mid 169.35446 91.836765) (end 169.3164 92.028107) (width 0.25) (layer "B.Cu") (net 18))
 (arc (start 172.281 88.649293) (mid 172.24294 88.840634) (end 172.134554 89.002846) (width 0.25) (layer "B.Cu") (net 18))
 (arc (start 172.281 85.899507) (mid 172.24294 85.708165) (end 172.134553 85.545953) (width 0.25) (layer "B.Cu") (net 18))
 (arc (start 169.845893 83.4644) (mid 170.037234 83.50246) (end 170.199446 83.610846) (width 0.25) (layer "B.Cu") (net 18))
 (arc (start 156.608621 73.007379) (mid 156.673506 72.964024) (end 156.750043 72.9488) (width 0.25) (layer "B.Cu") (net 18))
 (arc (start 165.608 82.313158) (mid 165.56994 82.121816) (end 165.461553 81.959604) (width 0.25) (layer "B.Cu") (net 18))
 (arc (start 166.108 83.4644) (mid 165.754447 83.317953) (end 165.608 82.9644) (width 0.25) (layer "B.Cu") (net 18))
 (arc (start 164.155 80.135707) (mid 164.11694 79.944365) (end 164.008553 79.782153) (width 0.25) (layer "B.Cu") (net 18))
 (arc (start 116.273422 68.521422) (mid 116.338307 68.564776) (end 116.414843 68.58) (width 0.25) (layer "B.Cu") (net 18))
 (arc (start 157.988 73.554493) (mid 158.02606 73.745834) (end 158.134446 73.908046) (width 0.25) (layer "B.Cu") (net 18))
 (arc (start 163.4826 106.24218) (mid 163.52066 106.433521) (end 163.629046 106.595733) (width 0.25) (layer "B.Cu") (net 18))
 (arc (start 104.709579 64.965421) (mid 104.644694 65.008776) (end 104.568157 65.024) (width 0.25) (layer "B.Cu") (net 18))
 (arc (start 111.132779 63.380779) (mid 111.067894 63.337424) (end 110.991357 63.3222) (width 0.25) (layer "B.Cu") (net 18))
 (arc (start 152.025821 73.793821) (mid 152.090706 73.837176) (end 152.167243 73.8524) (width 0.25) (layer "B.Cu") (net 18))
 (arc (start 164.155 80.445944) (mid 164.19306 80.637285) (end 164.301446 80.799497) (width 0.25) (layer "B.Cu") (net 18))
 (arc (start 126.042757 68.58) (mid 126.119294 68.595224) (end 126.184179 68.638579) (width 0.25) (layer "B.Cu") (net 18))
 (arc (start 83.394843 68.072) (mid 83.318307 68.087224) (end 83.253422 68.130578) (width 0.25) (layer "B.Cu") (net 18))
 (arc (start 82.166 69.300843) (mid 82.181224 69.224306) (end 82.224579 69.159421) (width 0.25) (layer "B.Cu") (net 18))
 (arc (start 155.822178 73.793822) (mid 155.757293 73.837176) (end 155.680757 73.8524) (width 0.25) (layer "B.Cu") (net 18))
 (arc (start 79.666 72.680177) (mid 79.650776 72.756713) (end 79.607422 72.821598) (width 0.25) (layer "B.Cu") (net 18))
 (arc (start 150.793157 72.644) (mid 150.869693 72.659224) (end 150.934578 72.702578) (width 0.25) (layer "B.Cu") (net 18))
 (arc (start 163.4826 105.379906) (mid 163.44454 105.188564) (end 163.336153 105.026352) (width 0.25) (layer "B.Cu") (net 18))
 (arc (start 73.8486 78.634243) (mid 73.863824 78.557706) (end 73.907179 78.492821) (width 0.25) (layer "B.Cu") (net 18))
 (segment (start 146.552047 64.801353) (end 147.452954 63.900446) (width 0.25) (layer "F.Cu") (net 24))
 (segment (start 146.9436 60.894543) (end 146.9436 58.39) (width 0.25) (layer "F.Cu") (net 24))
 (segment (start 149.311493 57.931447) (end 151.705046 60.325) (width 0.25) (layer "F.Cu") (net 24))
 (segment (start 147.5994 63.546893) (end 147.5994 61.964557) (width 0.25) (layer "F.Cu") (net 24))
 (segment (start 147.452953 61.611003) (end 147.090046 61.248096) (width 0.25) (layer "F.Cu") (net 24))
 (segment (start 146.4056 66.594893) (end 146.4056 65.154907) (width 0.25) (layer "F.Cu") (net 24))
 (segment (start 147.5486 67.945) (end 146.552046 66.948446) (width 0.25) (layer "F.Cu") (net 24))
 (segment (start 147.5486 57.785) (end 148.957939 57.785) (width 0.25) (layer "F.Cu") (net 24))
 (arc (start 147.452954 63.900446) (mid 147.56134 63.738234) (end 147.5994 63.546893) (width 0.25) (layer "F.Cu") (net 24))
 (arc (start 146.9436 60.894543) (mid 146.98166 61.085884) (end 147.090046 61.248096) (width 0.25) (layer "F.Cu") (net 24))
 (arc (start 146.552047 64.801353) (mid 146.44366 64.963565) (end 146.4056 65.154907) (width 0.25) (layer "F.Cu") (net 24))
 (arc (start 147.452953 61.611003) (mid 147.56134 61.773215) (end 147.5994 61.964557) (width 0.25) (layer "F.Cu") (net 24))
 (arc (start 146.4056 66.594893) (mid 146.44366 66.786234) (end 146.552046 66.948446) (width 0.25) (layer "F.Cu") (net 24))
 (arc (start 149.311493 57.931447) (mid 149.149281 57.82306) (end 148.957939 57.785) (width 0.25) (layer "F.Cu") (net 24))
 (segment (start 149.821493 67.945) (end 147.5486 67.945) (width 0.25) (layer "B.Cu") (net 24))
 (segment (start 152.5686 65.405) (end 150.175046 67.798554) (width 0.25) (layer "B.Cu") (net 24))
 (segment (start 142.908179 72.585421) (end 147.5486 67.945) (width 0.25) (layer "B.Cu") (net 24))
 (segment (start 141.388 72.644) (end 142.766757 72.644) (width 0.25) (layer "B.Cu") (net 24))
 (arc (start 150.175046 67.798554) (mid 150.012834 67.90694) (end 149.821493 67.945) (width 0.25) (layer "B.Cu") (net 24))
 (via (at 167.194701 104.57532) (size 0.8) (drill 0.4) (layers "F.Cu" "B.Cu") (free yes) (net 19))
 (via (at 170.688 95.7834) (size 0.8) (drill 0.4) (layers "F.Cu" "B.Cu") (free yes) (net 19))
 (via (at 172.0596 95.7834) (size 0.8) (drill 0.4) (layers "F.Cu" "B.Cu") (free yes) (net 20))
 (via (at 172.1612 104.6226) (size 0.8) (drill 0.4) (layers "F.Cu" "B.Cu") (free yes) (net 20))
 (via (at 166.5732 95.7834) (size 0.8) (drill 0.4) (layers "F.Cu" "B.Cu") (free yes) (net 16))
 (via (at 158.4452 104.648) (size 0.8) (drill 0.4) (layers "F.Cu" "B.Cu") (free yes) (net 16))
 (via (at 123.0376 87.9227) (size 0.8) (drill 0.4) (layers "F.Cu" "B.Cu") (free yes) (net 16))
 (via (at 167.9448 95.7834) (size 0.8) (drill 0.4) (layers "F.Cu" "B.Cu") (free yes) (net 17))
 (via (at 161.29 104.5972) (size 0.8) (drill 0.4) (layers "F.Cu" "B.Cu") (free yes) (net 17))
 (via (at 165.2016 95.7834) (size 0.8) (drill 0.4) (layers "F.Cu" "B.Cu") (free yes) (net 15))
 (via (at 157.415434 104.6226) (size 0.8) (drill 0.4) (layers "F.Cu" "B.Cu") (free yes) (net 15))
 (via (at 167.2844 74.2442) (size 0.8) (drill 0.4) (layers "F.Cu" "B.Cu") (free yes) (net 9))
 (via (at 162.541949 88.698049) (size 0.8) (drill 0.4) (layers "F.Cu" "B.Cu") (free yes) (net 7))
 (via (at 78.232 65.024) (size 0.8) (drill 0.4) (layers "F.Cu" "B.Cu") (free yes) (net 22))
 (via (at 153.416 122.428) (size 0.8) (drill 0.4) (layers "F.Cu" "B.Cu") (free yes) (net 22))
 (via (at 173.736 99.06) (size 0.8) (drill 0.4) (layers "F.Cu" "B.Cu") (free yes) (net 22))
 (via (at 120.4722 88.646) (size 0.8) (drill 0.4) (layers "F.Cu" "B.Cu") (free yes) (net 22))
 (via (at 170.18 97.536) (size 0.8) (drill 0.4) (layers "F.Cu" "B.Cu") (free yes) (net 22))
 (via (at 78.74 103.632) (size 0.8) (drill 0.4) (layers "F.Cu" "B.Cu") (free yes) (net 22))
 (via (at 162.8637 92.092422) (size 0.8) (drill 0.4) (layers "F.Cu" "B.Cu") (free yes) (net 22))
 (via (at 164.084 69.088) (size 0.8) (drill 0.4) (layers "F.Cu" "B.Cu") (free yes) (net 22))
 (via (at 136.144 73.66) (size 0.8) (drill 0.4) (layers "F.Cu" "B.Cu") (free yes) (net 22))
 (via (at 116.84 97.536) (size 0.8) (drill 0.4) (layers "F.Cu" "B.Cu") (free yes) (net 22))
 (via (at 154.432 76.708) (size 0.8) (drill 0.4) (layers "F.Cu" "B.Cu") (free yes) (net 22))
 (via (at 144.78 97.2058) (size 0.8) (drill 0.4) (layers "F.Cu" "B.Cu") (free yes) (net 22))
 (via (at 140.208 91.44) (size 0.8) (drill 0.4) (layers "F.Cu" "B.Cu") (free yes) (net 22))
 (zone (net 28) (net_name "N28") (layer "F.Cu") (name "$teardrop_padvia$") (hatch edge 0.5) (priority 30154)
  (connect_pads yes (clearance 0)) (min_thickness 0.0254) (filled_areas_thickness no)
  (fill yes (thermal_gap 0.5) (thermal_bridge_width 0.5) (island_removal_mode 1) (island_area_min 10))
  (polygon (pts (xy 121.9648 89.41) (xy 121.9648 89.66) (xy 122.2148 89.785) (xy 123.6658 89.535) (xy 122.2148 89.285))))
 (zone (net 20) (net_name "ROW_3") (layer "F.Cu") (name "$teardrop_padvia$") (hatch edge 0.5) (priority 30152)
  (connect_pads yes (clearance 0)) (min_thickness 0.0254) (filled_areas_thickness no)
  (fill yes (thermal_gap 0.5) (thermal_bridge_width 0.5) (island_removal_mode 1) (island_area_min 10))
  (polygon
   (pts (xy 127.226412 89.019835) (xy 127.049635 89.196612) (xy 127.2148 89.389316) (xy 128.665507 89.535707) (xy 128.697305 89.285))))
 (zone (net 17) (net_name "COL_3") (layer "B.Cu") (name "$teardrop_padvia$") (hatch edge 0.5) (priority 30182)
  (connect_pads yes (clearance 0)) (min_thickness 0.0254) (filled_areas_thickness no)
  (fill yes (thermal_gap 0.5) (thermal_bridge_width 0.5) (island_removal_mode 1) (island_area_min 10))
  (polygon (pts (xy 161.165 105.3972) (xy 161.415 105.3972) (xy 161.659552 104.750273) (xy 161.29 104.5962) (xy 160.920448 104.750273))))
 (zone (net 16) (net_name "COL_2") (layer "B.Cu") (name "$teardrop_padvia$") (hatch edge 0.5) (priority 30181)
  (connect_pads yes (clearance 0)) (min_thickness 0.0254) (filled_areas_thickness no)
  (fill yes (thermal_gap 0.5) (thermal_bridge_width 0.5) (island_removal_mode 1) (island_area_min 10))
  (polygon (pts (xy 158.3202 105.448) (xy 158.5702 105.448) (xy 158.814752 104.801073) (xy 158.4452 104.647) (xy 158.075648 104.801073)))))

